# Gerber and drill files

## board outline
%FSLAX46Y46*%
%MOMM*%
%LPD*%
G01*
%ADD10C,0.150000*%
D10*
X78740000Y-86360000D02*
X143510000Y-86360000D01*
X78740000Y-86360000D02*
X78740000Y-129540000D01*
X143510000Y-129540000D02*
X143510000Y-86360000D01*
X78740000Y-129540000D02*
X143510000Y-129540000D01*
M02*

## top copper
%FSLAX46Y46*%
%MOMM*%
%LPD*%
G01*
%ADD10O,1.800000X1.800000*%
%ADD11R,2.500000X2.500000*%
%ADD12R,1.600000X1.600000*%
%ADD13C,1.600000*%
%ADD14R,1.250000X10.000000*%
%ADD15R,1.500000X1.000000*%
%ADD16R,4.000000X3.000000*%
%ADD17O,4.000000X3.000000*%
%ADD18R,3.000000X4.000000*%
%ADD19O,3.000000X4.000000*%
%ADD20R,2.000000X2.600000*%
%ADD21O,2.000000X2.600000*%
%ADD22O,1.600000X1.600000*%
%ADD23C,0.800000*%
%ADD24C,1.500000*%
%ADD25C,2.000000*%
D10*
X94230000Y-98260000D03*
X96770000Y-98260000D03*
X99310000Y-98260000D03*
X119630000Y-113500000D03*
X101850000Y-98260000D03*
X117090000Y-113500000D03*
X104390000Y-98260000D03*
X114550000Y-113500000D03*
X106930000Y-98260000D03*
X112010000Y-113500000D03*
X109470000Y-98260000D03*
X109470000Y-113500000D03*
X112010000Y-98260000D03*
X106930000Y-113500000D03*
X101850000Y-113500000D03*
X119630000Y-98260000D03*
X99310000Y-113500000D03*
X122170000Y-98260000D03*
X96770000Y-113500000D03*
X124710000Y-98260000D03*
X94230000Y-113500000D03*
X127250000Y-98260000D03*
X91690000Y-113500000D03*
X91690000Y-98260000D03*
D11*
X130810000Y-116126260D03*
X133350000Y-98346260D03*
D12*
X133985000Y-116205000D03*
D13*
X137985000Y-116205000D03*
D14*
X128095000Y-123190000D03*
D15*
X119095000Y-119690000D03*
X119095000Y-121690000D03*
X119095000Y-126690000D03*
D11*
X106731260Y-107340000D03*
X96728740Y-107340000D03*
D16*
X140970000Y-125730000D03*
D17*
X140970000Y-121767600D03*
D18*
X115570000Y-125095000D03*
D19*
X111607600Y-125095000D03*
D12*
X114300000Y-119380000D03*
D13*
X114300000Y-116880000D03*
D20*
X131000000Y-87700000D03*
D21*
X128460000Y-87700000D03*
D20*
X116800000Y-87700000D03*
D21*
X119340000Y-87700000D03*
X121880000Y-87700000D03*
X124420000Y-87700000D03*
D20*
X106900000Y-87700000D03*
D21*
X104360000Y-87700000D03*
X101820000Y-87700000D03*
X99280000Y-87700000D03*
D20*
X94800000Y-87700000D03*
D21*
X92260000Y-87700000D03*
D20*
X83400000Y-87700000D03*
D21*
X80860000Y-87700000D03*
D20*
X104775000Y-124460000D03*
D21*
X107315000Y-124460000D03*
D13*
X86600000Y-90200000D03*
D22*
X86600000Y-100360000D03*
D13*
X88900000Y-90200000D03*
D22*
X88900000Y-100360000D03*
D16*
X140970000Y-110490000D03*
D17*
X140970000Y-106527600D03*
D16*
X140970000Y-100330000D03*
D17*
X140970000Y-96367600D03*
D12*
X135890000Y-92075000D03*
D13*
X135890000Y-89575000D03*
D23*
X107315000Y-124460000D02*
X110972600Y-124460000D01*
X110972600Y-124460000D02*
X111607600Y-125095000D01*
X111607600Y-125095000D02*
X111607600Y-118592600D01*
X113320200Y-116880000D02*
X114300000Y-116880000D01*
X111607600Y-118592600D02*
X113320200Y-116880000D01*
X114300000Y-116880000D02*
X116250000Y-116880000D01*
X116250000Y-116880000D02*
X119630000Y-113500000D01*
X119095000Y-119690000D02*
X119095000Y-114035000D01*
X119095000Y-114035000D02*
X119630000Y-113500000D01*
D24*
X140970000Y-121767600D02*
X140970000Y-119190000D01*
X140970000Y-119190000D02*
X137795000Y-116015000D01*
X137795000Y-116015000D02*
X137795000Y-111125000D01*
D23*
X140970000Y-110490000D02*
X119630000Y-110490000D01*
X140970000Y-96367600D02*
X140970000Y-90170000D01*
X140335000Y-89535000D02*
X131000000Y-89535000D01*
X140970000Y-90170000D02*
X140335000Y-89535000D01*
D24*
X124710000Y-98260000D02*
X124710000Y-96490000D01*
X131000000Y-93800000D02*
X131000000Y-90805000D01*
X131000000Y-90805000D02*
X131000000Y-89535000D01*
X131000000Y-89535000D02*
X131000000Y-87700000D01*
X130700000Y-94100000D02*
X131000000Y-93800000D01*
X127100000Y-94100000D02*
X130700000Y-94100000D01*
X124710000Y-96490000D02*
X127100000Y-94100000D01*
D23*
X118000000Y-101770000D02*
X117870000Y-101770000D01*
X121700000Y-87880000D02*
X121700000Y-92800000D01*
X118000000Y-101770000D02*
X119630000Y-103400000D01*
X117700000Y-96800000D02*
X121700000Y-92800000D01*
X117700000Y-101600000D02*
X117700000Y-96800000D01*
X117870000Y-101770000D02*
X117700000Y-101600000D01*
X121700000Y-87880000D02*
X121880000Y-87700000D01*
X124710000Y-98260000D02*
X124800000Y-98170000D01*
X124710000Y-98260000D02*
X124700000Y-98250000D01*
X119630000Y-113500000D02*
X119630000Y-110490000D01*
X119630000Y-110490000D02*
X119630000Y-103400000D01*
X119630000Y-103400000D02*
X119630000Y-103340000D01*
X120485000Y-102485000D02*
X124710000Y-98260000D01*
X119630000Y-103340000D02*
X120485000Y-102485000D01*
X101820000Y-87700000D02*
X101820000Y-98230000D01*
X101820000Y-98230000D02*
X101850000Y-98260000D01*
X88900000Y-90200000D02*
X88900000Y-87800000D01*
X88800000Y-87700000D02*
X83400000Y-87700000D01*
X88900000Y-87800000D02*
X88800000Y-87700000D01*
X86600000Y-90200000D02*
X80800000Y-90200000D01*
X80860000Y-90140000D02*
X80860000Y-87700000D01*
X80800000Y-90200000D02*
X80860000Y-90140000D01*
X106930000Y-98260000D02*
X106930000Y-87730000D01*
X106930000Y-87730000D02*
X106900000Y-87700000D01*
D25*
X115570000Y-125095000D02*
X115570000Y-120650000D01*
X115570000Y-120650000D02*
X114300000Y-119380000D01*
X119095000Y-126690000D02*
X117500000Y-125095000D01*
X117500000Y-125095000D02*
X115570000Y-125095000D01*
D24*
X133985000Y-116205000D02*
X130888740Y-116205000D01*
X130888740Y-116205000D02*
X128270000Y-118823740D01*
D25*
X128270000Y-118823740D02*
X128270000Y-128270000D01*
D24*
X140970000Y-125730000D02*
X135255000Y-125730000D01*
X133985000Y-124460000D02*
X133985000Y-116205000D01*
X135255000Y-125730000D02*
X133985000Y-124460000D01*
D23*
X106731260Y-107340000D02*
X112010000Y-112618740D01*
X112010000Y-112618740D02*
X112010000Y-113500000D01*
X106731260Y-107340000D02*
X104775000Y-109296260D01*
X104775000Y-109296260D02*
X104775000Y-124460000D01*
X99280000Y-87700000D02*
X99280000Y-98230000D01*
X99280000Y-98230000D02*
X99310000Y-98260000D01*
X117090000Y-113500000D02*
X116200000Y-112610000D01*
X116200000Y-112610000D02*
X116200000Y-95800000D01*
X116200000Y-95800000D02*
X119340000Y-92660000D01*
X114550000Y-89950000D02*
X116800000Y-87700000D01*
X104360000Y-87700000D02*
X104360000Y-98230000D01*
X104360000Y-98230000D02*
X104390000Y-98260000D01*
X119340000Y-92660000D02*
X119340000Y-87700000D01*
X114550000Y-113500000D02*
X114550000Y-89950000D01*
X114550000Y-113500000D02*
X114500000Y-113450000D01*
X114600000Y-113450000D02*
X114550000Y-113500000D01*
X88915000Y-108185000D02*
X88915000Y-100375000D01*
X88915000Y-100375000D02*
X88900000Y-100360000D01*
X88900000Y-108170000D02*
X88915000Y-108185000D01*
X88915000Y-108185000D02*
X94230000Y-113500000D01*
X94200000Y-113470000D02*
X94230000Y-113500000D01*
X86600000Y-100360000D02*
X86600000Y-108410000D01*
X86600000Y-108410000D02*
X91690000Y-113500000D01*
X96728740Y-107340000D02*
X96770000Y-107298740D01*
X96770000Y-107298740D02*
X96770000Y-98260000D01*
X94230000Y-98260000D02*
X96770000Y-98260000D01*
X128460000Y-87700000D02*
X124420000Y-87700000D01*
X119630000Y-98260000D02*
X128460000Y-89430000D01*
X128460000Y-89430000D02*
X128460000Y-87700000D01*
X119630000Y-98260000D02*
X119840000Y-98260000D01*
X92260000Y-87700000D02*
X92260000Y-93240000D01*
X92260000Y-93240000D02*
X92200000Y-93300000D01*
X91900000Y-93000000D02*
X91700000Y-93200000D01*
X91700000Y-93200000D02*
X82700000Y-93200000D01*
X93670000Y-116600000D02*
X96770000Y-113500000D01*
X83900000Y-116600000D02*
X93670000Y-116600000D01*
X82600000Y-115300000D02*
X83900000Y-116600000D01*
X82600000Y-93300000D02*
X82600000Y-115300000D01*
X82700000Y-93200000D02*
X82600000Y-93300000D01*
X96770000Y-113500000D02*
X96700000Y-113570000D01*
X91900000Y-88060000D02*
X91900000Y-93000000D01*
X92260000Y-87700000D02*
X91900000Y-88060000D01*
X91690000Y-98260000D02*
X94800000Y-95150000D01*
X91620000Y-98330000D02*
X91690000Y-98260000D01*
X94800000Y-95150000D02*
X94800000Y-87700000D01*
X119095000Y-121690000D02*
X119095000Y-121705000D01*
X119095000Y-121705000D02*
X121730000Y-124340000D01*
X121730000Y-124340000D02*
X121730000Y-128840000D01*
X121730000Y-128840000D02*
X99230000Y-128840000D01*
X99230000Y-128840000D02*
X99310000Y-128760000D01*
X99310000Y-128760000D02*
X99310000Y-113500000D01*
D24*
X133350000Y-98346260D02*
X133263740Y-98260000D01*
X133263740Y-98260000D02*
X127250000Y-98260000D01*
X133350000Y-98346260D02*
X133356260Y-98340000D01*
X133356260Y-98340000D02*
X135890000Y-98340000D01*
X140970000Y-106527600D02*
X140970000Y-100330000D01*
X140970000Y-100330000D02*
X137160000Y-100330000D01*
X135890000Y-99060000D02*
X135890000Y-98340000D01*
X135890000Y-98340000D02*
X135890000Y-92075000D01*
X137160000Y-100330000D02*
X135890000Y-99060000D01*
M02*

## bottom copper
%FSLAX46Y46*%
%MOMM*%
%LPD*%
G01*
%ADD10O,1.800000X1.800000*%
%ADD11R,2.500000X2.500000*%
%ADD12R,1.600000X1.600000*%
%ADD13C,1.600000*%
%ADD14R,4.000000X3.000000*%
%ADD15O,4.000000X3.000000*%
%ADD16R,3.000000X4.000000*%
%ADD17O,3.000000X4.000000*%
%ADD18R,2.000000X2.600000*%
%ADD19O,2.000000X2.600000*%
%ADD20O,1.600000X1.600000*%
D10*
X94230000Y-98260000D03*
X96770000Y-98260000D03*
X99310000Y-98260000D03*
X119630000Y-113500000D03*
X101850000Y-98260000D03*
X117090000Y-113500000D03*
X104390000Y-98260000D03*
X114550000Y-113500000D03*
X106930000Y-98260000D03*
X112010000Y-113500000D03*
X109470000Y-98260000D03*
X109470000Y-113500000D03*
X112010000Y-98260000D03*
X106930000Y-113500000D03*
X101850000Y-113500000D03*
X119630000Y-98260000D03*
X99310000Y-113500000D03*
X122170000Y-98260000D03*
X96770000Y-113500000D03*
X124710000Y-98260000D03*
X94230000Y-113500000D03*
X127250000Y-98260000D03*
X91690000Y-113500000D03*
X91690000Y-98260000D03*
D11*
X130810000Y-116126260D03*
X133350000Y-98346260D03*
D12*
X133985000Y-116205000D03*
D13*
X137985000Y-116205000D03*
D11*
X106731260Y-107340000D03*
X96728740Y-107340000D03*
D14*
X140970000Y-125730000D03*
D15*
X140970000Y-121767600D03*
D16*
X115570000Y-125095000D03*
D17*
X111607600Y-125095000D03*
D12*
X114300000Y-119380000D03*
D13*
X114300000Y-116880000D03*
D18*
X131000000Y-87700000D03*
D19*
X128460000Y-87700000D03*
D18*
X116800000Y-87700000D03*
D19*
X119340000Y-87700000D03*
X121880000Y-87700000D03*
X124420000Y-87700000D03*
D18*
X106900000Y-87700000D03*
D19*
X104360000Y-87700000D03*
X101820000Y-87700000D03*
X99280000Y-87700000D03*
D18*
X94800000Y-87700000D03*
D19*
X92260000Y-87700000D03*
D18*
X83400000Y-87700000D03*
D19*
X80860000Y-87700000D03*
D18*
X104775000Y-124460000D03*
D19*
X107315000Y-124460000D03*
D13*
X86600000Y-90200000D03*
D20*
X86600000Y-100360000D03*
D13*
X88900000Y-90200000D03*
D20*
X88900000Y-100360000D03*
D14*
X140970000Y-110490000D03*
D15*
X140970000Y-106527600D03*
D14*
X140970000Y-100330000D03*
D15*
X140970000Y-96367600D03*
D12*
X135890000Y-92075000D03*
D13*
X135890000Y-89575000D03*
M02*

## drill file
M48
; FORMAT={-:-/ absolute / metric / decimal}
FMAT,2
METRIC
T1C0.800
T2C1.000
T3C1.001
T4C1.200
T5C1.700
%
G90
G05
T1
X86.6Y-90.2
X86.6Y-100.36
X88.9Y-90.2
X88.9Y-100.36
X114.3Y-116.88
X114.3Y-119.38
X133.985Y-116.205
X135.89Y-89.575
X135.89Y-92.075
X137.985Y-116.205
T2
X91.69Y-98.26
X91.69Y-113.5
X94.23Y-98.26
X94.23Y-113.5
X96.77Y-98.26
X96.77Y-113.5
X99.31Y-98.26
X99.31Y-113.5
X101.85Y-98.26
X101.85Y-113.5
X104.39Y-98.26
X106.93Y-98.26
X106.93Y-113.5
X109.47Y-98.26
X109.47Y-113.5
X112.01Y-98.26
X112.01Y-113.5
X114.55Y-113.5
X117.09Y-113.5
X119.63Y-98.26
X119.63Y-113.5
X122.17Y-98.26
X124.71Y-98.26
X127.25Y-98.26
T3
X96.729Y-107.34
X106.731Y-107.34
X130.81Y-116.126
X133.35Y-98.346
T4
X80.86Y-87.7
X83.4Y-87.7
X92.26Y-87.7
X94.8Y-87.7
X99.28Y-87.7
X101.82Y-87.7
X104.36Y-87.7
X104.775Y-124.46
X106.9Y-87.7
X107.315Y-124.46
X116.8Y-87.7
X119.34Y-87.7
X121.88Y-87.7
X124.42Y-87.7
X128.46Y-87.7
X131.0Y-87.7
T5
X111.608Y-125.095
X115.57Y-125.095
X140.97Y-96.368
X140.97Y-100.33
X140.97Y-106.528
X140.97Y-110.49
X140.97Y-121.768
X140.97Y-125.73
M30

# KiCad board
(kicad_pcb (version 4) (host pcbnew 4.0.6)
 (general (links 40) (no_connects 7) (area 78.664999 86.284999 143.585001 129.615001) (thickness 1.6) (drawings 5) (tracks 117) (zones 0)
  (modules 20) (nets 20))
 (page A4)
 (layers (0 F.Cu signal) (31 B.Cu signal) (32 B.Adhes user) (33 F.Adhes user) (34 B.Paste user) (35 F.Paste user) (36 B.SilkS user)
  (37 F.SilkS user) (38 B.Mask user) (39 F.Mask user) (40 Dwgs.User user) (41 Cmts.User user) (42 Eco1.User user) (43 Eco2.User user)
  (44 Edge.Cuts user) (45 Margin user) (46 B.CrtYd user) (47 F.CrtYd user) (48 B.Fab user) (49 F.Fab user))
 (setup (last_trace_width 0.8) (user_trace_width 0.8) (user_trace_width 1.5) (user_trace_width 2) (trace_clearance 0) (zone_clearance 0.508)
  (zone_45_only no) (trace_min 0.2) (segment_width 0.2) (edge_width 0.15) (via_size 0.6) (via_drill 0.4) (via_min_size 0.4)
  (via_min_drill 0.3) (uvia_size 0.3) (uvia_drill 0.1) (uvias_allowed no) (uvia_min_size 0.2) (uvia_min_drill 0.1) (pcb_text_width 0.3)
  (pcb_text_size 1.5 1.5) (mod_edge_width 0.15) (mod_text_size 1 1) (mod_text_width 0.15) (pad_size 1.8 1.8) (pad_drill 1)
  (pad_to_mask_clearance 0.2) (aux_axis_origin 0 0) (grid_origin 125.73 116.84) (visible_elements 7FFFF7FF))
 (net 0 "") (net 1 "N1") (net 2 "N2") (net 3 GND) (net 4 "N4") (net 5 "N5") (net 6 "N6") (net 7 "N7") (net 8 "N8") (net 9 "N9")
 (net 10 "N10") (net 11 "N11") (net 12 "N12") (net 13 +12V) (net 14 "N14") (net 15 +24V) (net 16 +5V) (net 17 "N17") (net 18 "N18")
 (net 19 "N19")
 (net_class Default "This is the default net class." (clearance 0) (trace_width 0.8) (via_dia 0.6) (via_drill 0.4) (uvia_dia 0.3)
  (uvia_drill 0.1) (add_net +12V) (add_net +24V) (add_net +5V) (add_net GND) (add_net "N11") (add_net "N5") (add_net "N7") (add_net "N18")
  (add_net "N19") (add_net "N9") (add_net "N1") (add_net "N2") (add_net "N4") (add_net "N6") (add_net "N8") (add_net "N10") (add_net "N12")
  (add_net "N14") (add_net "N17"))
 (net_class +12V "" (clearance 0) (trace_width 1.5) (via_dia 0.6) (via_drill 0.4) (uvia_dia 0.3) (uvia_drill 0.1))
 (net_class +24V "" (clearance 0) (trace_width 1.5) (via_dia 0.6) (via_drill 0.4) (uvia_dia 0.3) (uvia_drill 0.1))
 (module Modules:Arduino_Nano (layer B.Cu) (at 127.25 113.5 90)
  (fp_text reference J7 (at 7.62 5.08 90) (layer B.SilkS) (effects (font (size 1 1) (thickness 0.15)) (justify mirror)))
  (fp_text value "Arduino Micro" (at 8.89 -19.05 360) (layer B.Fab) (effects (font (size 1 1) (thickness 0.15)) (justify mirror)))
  (pad 3.3V thru_hole oval (at 15.24 -33.02 90) (size 1.8 1.8) (drill 1) (layers *.Cu *.Mask) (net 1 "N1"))
  (pad AREF thru_hole oval (at 15.24 -30.48 90) (size 1.8 1.8) (drill 1) (layers *.Cu *.Mask) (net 1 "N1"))
  (pad A0 thru_hole oval (at 15.24 -27.94 90) (size 1.8 1.8) (drill 1) (layers *.Cu *.Mask) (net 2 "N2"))
  (pad GND thru_hole oval (at 0 -7.62 90) (size 1.8 1.8) (drill 1) (layers *.Cu *.Mask) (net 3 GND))
  (pad A1 thru_hole oval (at 15.24 -25.4 90) (size 1.8 1.8) (drill 1) (layers *.Cu *.Mask) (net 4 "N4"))
  (pad SDA thru_hole oval (at 0 -10.16 90) (size 1.8 1.8) (drill 1) (layers *.Cu *.Mask) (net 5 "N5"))
  (pad A2 thru_hole oval (at 15.24 -22.86 90) (size 1.8 1.8) (drill 1) (layers *.Cu *.Mask) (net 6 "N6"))
  (pad SCL thru_hole oval (at 0 -12.7 90) (size 1.8 1.8) (drill 1) (layers *.Cu *.Mask) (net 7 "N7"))
  (pad A3 thru_hole oval (at 15.24 -20.32 90) (size 1.8 1.8) (drill 1) (layers *.Cu *.Mask) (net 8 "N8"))
  (pad D4 thru_hole oval (at 0 -15.24 90) (size 1.8 1.8) (drill 1) (layers *.Cu *.Mask) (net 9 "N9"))
  (pad A4 thru_hole oval (at 15.24 -17.78 90) (size 1.8 1.8) (drill 1) (layers *.Cu *.Mask) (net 9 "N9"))
  (pad D5 thru_hole oval (at 0 -17.78 90) (size 1.8 1.8) (drill 1) (layers *.Cu *.Mask))
  (pad A5 thru_hole oval (at 15.24 -15.24 90) (size 1.8 1.8) (drill 1) (layers *.Cu *.Mask) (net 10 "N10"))
  (pad D6 thru_hole oval (at 0 -20.32 90) (size 1.8 1.8) (drill 1) (layers *.Cu *.Mask))
  (pad D8 thru_hole oval (at 0 -25.4 90) (size 1.8 1.8) (drill 1) (layers *.Cu *.Mask))
  (pad 5v thru_hole oval (at 15.24 -7.62 90) (size 1.8 1.8) (drill 1) (layers *.Cu *.Mask))
  (pad D9 thru_hole oval (at 0 -27.94 90) (size 1.8 1.8) (drill 1) (layers *.Cu *.Mask) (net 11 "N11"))
  (pad RS thru_hole oval (at 15.24 -5.08 90) (size 1.8 1.8) (drill 1) (layers *.Cu *.Mask))
  (pad D10 thru_hole oval (at 0 -30.48 90) (size 1.8 1.8) (drill 1) (layers *.Cu *.Mask))
  (pad GND thru_hole oval (at 15.24 -2.54 90) (size 1.8 1.8) (drill 1) (layers *.Cu *.Mask) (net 3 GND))
  (pad D11 thru_hole oval (at 0 -33.02 90) (size 1.8 1.8) (drill 1) (layers *.Cu *.Mask) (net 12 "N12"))
  (pad Vin thru_hole oval (at 15.24 0 90) (size 1.8 1.8) (drill 1) (layers *.Cu *.Mask) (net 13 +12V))
  (pad D12 thru_hole oval (at 0 -35.56 90) (size 1.8 1.8) (drill 1) (layers *.Cu *.Mask) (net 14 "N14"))
  (pad D13 thru_hole oval (at 15.24 -35.56 90) (size 1.8 1.8) (drill 1) (layers *.Cu *.Mask)))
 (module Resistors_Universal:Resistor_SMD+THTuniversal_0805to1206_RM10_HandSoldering (layer F.Cu) (at 130.81 111.125 90)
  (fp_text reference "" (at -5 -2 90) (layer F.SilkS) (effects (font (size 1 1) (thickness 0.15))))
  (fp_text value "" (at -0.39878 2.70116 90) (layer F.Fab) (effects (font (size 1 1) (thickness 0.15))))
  (pad 1 thru_hole rect (at -5.00126 0 270) (size 2.5 2.5) (drill 1.00076) (layers *.Cu *.Mask) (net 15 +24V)))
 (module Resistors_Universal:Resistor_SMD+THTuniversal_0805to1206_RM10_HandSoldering (layer F.Cu) (at 133.35 93.345 90)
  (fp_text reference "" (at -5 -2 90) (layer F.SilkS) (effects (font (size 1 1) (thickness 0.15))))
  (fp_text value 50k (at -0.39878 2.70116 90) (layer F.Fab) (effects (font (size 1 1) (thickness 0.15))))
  (pad 1 thru_hole rect (at -5.00126 0 270) (size 2.5 2.5) (drill 1.00076) (layers *.Cu *.Mask) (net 13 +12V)))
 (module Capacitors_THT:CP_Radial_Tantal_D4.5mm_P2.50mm (layer B.Cu) (at 133.985 116.205)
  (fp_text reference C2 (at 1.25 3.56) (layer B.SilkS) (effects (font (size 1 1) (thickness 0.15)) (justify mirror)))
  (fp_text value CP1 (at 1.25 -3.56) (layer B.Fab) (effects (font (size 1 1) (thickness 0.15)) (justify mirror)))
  (pad 1 thru_hole rect (at 0 0) (size 1.6 1.6) (drill 0.8) (layers *.Cu *.Mask) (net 15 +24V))
  (pad 2 thru_hole circle (at 4 0) (size 1.6 1.6) (drill 0.8) (layers *.Cu *.Mask) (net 3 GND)))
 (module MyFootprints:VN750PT (layer F.Cu) (at 125.095 123.19 270)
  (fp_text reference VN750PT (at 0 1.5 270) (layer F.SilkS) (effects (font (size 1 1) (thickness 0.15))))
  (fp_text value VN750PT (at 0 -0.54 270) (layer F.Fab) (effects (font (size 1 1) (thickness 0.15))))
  (pad Vcc smd rect (at 0 -3 270) (size 10 1.25) (layers F.Cu F.Paste F.Mask) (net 15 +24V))
  (pad GND smd rect (at -3.5 6 270) (size 1 1.5) (layers F.Cu F.Paste F.Mask) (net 3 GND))
  (pad Inpu smd rect (at -1.5 6 270) (size 1 1.5) (layers F.Cu F.Paste F.Mask) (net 11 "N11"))
  (pad Vout smd rect (at 3.5 6 270) (size 1 1.5) (layers F.Cu F.Paste F.Mask) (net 15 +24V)))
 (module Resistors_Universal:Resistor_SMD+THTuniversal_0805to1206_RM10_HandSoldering (layer F.Cu) (at 101.73 107.34 180)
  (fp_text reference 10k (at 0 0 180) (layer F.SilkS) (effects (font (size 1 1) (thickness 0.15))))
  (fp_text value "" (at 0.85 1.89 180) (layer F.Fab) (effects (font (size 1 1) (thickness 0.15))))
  (pad 1 thru_hole rect (at -5.00126 0) (size 2.5 2.5) (drill 1.00076) (layers *.Cu *.Mask) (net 9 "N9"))
  (pad 2 thru_hole rect (at 5.00126 0) (size 2.5 2.5) (drill 1.00076) (layers *.Cu *.Mask) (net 1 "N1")))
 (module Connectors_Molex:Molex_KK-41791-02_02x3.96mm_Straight (layer F.Cu) (at 140.97 125.73 90)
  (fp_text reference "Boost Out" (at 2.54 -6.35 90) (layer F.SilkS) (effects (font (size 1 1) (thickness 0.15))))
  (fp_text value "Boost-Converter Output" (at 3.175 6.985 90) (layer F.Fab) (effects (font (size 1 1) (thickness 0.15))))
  (pad 1 thru_hole rect (at 0 0 90) (size 3 4) (drill 1.7) (layers *.Cu *.Mask) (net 15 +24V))
  (pad 2 thru_hole oval (at 3.9624 0 90) (size 3 4) (drill 1.7) (layers *.Cu *.Mask) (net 3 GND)))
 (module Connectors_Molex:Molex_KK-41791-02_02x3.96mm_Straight (layer F.Cu) (at 115.57 125.095 180)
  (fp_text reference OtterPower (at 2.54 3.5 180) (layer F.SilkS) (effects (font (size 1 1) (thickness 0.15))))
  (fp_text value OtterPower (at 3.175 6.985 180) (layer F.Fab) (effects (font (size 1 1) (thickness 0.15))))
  (pad 1 thru_hole rect (at 0 0 180) (size 3 4) (drill 1.7) (layers *.Cu *.Mask) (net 15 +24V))
  (pad 2 thru_hole oval (at 3.9624 0 180) (size 3 4) (drill 1.7) (layers *.Cu *.Mask) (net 3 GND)))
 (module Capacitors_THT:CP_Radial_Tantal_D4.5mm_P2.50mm (layer B.Cu) (at 114.3 119.38 90)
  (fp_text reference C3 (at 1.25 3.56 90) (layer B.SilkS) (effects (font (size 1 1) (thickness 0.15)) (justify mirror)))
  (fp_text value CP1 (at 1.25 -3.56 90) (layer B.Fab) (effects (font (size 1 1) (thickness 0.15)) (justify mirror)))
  (pad + thru_hole rect (at 0 0 90) (size 1.6 1.6) (drill 0.8) (layers *.Cu *.Mask) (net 15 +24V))
  (pad 2 thru_hole circle (at 2.5 0 90) (size 1.6 1.6) (drill 0.8) (layers *.Cu *.Mask) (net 3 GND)))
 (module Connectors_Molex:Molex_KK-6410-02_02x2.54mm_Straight (layer F.Cu) (at 131 87.7 180)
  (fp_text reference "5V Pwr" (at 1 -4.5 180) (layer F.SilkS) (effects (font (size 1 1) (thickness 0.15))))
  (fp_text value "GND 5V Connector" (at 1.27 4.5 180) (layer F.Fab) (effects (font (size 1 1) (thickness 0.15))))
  (pad 1 thru_hole rect (at 0 0 180) (size 2 2.6) (drill 1.2) (layers *.Cu *.Mask) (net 3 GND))
  (pad 2 thru_hole oval (at 2.54 0 180) (size 2 2.6) (drill 1.2) (layers *.Cu *.Mask) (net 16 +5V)))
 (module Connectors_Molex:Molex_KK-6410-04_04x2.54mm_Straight (layer F.Cu) (at 116.8 87.7)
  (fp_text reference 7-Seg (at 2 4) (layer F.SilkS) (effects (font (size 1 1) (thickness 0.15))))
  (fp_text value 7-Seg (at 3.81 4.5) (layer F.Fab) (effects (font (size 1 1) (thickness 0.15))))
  (pad 1 thru_hole rect (at 0 0) (size 2 2.6) (drill 1.2) (layers *.Cu *.Mask) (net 5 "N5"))
  (pad 2 thru_hole oval (at 2.54 0) (size 2 2.6) (drill 1.2) (layers *.Cu *.Mask) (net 7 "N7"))
  (pad 3 thru_hole oval (at 5.08 0) (size 2 2.6) (drill 1.2) (layers *.Cu *.Mask) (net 3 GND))
  (pad 4 thru_hole oval (at 7.62 0) (size 2 2.6) (drill 1.2) (layers *.Cu *.Mask) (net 16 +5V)))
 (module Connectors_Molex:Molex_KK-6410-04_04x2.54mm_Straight (layer F.Cu) (at 106.9 87.7 180)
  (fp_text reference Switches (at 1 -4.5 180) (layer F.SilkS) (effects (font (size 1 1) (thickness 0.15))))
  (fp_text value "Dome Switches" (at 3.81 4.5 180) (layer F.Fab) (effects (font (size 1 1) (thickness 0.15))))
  (pad 1 thru_hole rect (at 0 0 180) (size 2 2.6) (drill 1.2) (layers *.Cu *.Mask) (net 8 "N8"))
  (pad 2 thru_hole oval (at 2.54 0 180) (size 2 2.6) (drill 1.2) (layers *.Cu *.Mask) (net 6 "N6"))
  (pad 3 thru_hole oval (at 5.08 0 180) (size 2 2.6) (drill 1.2) (layers *.Cu *.Mask) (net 4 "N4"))
  (pad 4 thru_hole oval (at 7.62 0 180) (size 2 2.6) (drill 1.2) (layers *.Cu *.Mask) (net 2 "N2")))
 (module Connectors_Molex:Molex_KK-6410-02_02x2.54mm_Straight (layer F.Cu) (at 94.8 87.7 180)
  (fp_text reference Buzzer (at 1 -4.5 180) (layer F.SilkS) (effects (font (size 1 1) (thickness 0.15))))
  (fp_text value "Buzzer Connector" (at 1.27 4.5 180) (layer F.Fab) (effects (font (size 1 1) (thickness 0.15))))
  (pad 1 thru_hole rect (at 0 0 180) (size 2 2.6) (drill 1.2) (layers *.Cu *.Mask) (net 10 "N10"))
  (pad 2 thru_hole oval (at 2.54 0 180) (size 2 2.6) (drill 1.2) (layers *.Cu *.Mask) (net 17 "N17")))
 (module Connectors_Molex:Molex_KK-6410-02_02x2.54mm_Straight (layer F.Cu) (at 83.4 87.7 180)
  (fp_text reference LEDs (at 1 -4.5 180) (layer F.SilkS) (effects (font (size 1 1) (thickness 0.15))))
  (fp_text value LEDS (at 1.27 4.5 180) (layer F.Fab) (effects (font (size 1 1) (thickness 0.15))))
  (pad 1 thru_hole rect (at 0 0 180) (size 2 2.6) (drill 1.2) (layers *.Cu *.Mask) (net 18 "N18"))
  (pad 2 thru_hole oval (at 2.54 0 180) (size 2 2.6) (drill 1.2) (layers *.Cu *.Mask) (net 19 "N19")))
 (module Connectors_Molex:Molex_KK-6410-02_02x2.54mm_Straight (layer F.Cu) (at 104.775 124.46)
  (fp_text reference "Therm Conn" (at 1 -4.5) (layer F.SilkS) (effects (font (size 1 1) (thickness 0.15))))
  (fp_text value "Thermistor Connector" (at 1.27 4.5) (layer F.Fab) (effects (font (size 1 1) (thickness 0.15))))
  (pad 1 thru_hole rect (at 0 0) (size 2 2.6) (drill 1.2) (layers *.Cu *.Mask) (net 9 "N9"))
  (pad 2 thru_hole oval (at 2.54 0) (size 2 2.6) (drill 1.2) (layers *.Cu *.Mask) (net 3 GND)))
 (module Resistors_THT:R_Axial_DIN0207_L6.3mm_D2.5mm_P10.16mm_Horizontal (layer F.Cu) (at 86.6 90.2 270)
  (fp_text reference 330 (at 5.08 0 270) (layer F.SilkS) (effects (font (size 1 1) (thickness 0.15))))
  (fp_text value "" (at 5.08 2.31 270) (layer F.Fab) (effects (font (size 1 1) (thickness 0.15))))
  (pad 1 thru_hole circle (at 0 0 270) (size 1.6 1.6) (drill 0.8) (layers *.Cu *.Mask) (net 19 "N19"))
  (pad 2 thru_hole oval (at 10.16 0 270) (size 1.6 1.6) (drill 0.8) (layers *.Cu *.Mask) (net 14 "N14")))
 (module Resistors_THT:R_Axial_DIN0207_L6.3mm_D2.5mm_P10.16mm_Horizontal (layer F.Cu) (at 88.9 90.2 270)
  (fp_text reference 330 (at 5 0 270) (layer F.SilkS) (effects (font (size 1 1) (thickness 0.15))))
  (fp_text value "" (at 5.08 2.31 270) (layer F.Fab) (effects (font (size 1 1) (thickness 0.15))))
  (pad 1 thru_hole circle (at 0 0 270) (size 1.6 1.6) (drill 0.8) (layers *.Cu *.Mask) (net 18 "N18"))
  (pad 2 thru_hole oval (at 10.16 0 270) (size 1.6 1.6) (drill 0.8) (layers *.Cu *.Mask) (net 12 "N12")))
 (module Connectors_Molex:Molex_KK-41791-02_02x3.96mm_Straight (layer F.Cu) (at 140.97 110.49 90)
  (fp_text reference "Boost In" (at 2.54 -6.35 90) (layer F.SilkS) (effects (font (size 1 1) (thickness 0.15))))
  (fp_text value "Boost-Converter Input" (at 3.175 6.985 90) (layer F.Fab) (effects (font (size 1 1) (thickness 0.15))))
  (pad 1 thru_hole rect (at 0 0 90) (size 3 4) (drill 1.7) (layers *.Cu *.Mask) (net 3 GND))
  (pad 2 thru_hole oval (at 3.9624 0 90) (size 3 4) (drill 1.7) (layers *.Cu *.Mask) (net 13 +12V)))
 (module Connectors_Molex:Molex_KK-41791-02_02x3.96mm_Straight (layer F.Cu) (at 140.97 100.33 90)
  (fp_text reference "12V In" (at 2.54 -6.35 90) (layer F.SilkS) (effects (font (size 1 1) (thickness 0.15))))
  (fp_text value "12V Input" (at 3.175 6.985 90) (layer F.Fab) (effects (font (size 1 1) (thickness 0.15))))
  (pad 1 thru_hole rect (at 0 0 90) (size 3 4) (drill 1.7) (layers *.Cu *.Mask) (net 13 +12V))
  (pad 2 thru_hole oval (at 3.9624 0 90) (size 3 4) (drill 1.7) (layers *.Cu *.Mask) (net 3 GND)))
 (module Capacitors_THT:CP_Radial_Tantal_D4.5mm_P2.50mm (layer F.Cu) (at 135.89 92.075 90)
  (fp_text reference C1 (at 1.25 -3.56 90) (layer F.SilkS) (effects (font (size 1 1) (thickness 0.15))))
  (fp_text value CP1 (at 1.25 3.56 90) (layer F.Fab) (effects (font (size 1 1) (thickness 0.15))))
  (pad 1 thru_hole rect (at 0 0 90) (size 1.6 1.6) (drill 0.8) (layers *.Cu *.Mask) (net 13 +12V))
  (pad 2 thru_hole circle (at 2.5 0 90) (size 1.6 1.6) (drill 0.8) (layers *.Cu *.Mask) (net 3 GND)))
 (gr_line (start 78.74 86.36) (end 143.51 86.36) (angle 90) (layer Edge.Cuts) (width 0.15))
 (gr_line (start 78.74 86.36) (end 78.74 129.54) (angle 90) (layer Edge.Cuts) (width 0.15))
 (gr_line (start 143.51 129.54) (end 143.51 86.36) (angle 90) (layer Edge.Cuts) (width 0.15))
 (gr_line (start 78.74 129.54) (end 143.51 129.54) (angle 90) (layer Edge.Cuts) (width 0.15))
 (segment (start 107.315 124.46) (end 110.9726 124.46) (width 0.8) (layer F.Cu) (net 3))
 (segment (start 110.9726 124.46) (end 111.6076 125.095) (width 0.8) (layer F.Cu) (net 3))
 (segment (start 111.6076 125.095) (end 111.6076 118.5926) (width 0.8) (layer F.Cu) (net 3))
 (segment (start 113.3202 116.88) (end 114.3 116.88) (width 0.8) (layer F.Cu) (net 3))
 (segment (start 111.6076 118.5926) (end 113.3202 116.88) (width 0.8) (layer F.Cu) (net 3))
 (segment (start 114.3 116.88) (end 116.25 116.88) (width 0.8) (layer F.Cu) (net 3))
 (segment (start 116.25 116.88) (end 119.63 113.5) (width 0.8) (layer F.Cu) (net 3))
 (segment (start 119.095 119.69) (end 119.095 114.035) (width 0.8) (layer F.Cu) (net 3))
 (segment (start 119.095 114.035) (end 119.63 113.5) (width 0.8) (layer F.Cu) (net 3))
 (segment (start 140.97 121.7676) (end 140.97 119.19) (width 1.5) (layer F.Cu) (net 3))
 (segment (start 140.97 119.19) (end 137.795 116.015) (width 1.5) (layer F.Cu) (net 3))
 (segment (start 137.795 116.015) (end 137.795 111.125) (width 1.5) (layer F.Cu) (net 3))
 (segment (start 140.97 110.49) (end 119.63 110.49) (width 0.8) (layer F.Cu) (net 3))
 (segment (start 140.97 96.3676) (end 140.97 90.17) (width 0.8) (layer F.Cu) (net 3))
 (segment (start 140.335 89.535) (end 131 89.535) (width 0.8) (layer F.Cu) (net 3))
 (segment (start 140.97 90.17) (end 140.335 89.535) (width 0.8) (layer F.Cu) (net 3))
 (segment (start 124.71 98.26) (end 124.71 96.49) (width 1.5) (layer F.Cu) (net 3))
 (segment (start 131 93.8) (end 131 90.805) (width 1.5) (layer F.Cu) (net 3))
 (segment (start 131 90.805) (end 131 89.535) (width 1.5) (layer F.Cu) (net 3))
 (segment (start 131 89.535) (end 131 87.7) (width 1.5) (layer F.Cu) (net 3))
 (segment (start 130.7 94.1) (end 131 93.8) (width 1.5) (layer F.Cu) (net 3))
 (segment (start 127.1 94.1) (end 130.7 94.1) (width 1.5) (layer F.Cu) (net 3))
 (segment (start 124.71 96.49) (end 127.1 94.1) (width 1.5) (layer F.Cu) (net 3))
 (segment (start 118 101.77) (end 117.87 101.77) (width 0.8) (layer F.Cu) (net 3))
 (segment (start 121.7 87.88) (end 121.7 92.8) (width 0.8) (layer F.Cu) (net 3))
 (segment (start 118 101.77) (end 119.63 103.4) (width 0.8) (layer F.Cu) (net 3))
 (segment (start 117.7 96.8) (end 121.7 92.8) (width 0.8) (layer F.Cu) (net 3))
 (segment (start 117.7 101.6) (end 117.7 96.8) (width 0.8) (layer F.Cu) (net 3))
 (segment (start 117.87 101.77) (end 117.7 101.6) (width 0.8) (layer F.Cu) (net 3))
 (segment (start 121.7 87.88) (end 121.88 87.7) (width 0.8) (layer F.Cu) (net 3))
 (segment (start 124.71 98.26) (end 124.8 98.17) (width 0.8) (layer F.Cu) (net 3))
 (segment (start 124.71 98.26) (end 124.7 98.25) (width 0.8) (layer F.Cu) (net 3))
 (segment (start 119.63 113.5) (end 119.63 110.49) (width 0.8) (layer F.Cu) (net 3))
 (segment (start 119.63 110.49) (end 119.63 103.4) (width 0.8) (layer F.Cu) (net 3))
 (segment (start 119.63 103.4) (end 119.63 103.34) (width 0.8) (layer F.Cu) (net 3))
 (segment (start 120.485 102.485) (end 124.71 98.26) (width 0.8) (layer F.Cu) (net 3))
 (segment (start 119.63 103.34) (end 120.485 102.485) (width 0.8) (layer F.Cu) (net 3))
 (segment (start 101.82 87.7) (end 101.82 98.23) (width 0.8) (layer F.Cu) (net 4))
 (segment (start 101.82 98.23) (end 101.85 98.26) (width 0.8) (layer F.Cu) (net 4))
 (segment (start 88.9 90.2) (end 88.9 87.8) (width 0.8) (layer F.Cu) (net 18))
 (segment (start 88.8 87.7) (end 83.4 87.7) (width 0.8) (layer F.Cu) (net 18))
 (segment (start 88.9 87.8) (end 88.8 87.7) (width 0.8) (layer F.Cu) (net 18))
 (segment (start 86.6 90.2) (end 80.8 90.2) (width 0.8) (layer F.Cu) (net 19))
 (segment (start 80.86 90.14) (end 80.86 87.7) (width 0.8) (layer F.Cu) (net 19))
 (segment (start 80.8 90.2) (end 80.86 90.14) (width 0.8) (layer F.Cu) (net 19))
 (segment (start 106.93 98.26) (end 106.93 87.73) (width 0.8) (layer F.Cu) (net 8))
 (segment (start 106.93 87.73) (end 106.9 87.7) (width 0.8) (layer F.Cu) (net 8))
 (segment (start 115.57 125.095) (end 115.57 120.65) (width 2) (layer F.Cu) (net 15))
 (segment (start 115.57 120.65) (end 114.3 119.38) (width 2) (layer F.Cu) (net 15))
 (segment (start 119.095 126.69) (end 117.5 125.095) (width 2) (layer F.Cu) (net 15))
 (segment (start 117.5 125.095) (end 115.57 125.095) (width 2) (layer F.Cu) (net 15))
 (segment (start 133.985 116.205) (end 130.88874 116.205) (width 1.5) (layer F.Cu) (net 15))
 (segment (start 130.88874 116.205) (end 128.27 118.82374) (width 1.5) (layer F.Cu) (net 15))
 (segment (start 128.27 118.82374) (end 128.27 128.27) (width 2) (layer F.Cu) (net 15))
 (segment (start 140.97 125.73) (end 135.255 125.73) (width 1.5) (layer F.Cu) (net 15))
 (segment (start 133.985 124.46) (end 133.985 116.205) (width 1.5) (layer F.Cu) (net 15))
 (segment (start 135.255 125.73) (end 133.985 124.46) (width 1.5) (layer F.Cu) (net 15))
 (segment (start 106.73126 107.34) (end 112.01 112.61874) (width 0.8) (layer F.Cu) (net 9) (status C00000))
 (segment (start 112.01 112.61874) (end 112.01 113.5) (width 0.8) (layer F.Cu) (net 9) (status C00000))
 (segment (start 106.73126 107.34) (end 104.775 109.29626) (width 0.8) (layer F.Cu) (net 9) (status 400000))
 (segment (start 104.775 109.29626) (end 104.775 124.46) (width 0.8) (layer F.Cu) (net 9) (status 800000))
 (segment (start 99.28 87.7) (end 99.28 98.23) (width 0.8) (layer F.Cu) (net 2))
 (segment (start 99.28 98.23) (end 99.31 98.26) (width 0.8) (layer F.Cu) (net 2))
 (segment (start 117.09 113.5) (end 116.2 112.61) (width 0.8) (layer F.Cu) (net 5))
 (segment (start 116.2 112.61) (end 116.2 95.8) (width 0.8) (layer F.Cu) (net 5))
 (segment (start 116.2 95.8) (end 119.34 92.66) (width 0.8) (layer F.Cu) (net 5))
 (segment (start 114.55 89.95) (end 116.8 87.7) (width 0.8) (layer F.Cu) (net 5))
 (segment (start 104.36 87.7) (end 104.36 98.23) (width 0.8) (layer F.Cu) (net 6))
 (segment (start 104.36 98.23) (end 104.39 98.26) (width 0.8) (layer F.Cu) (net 6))
 (segment (start 119.34 92.66) (end 119.34 87.7) (width 0.8) (layer F.Cu) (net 7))
 (segment (start 114.55 113.5) (end 114.55 89.95) (width 0.8) (layer F.Cu) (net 7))
 (segment (start 114.55 113.5) (end 114.5 113.45) (width 0.8) (layer F.Cu) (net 7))
 (segment (start 114.6 113.45) (end 114.55 113.5) (width 0.8) (layer F.Cu) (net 7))
 (segment (start 88.915 108.185) (end 88.915 100.375) (width 0.8) (layer F.Cu) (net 12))
 (segment (start 88.915 100.375) (end 88.9 100.36) (width 0.8) (layer F.Cu) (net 12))
 (segment (start 88.9 108.17) (end 88.915 108.185) (width 0.8) (layer F.Cu) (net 12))
 (segment (start 88.915 108.185) (end 94.23 113.5) (width 0.8) (layer F.Cu) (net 12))
 (segment (start 94.2 113.47) (end 94.23 113.5) (width 0.8) (layer F.Cu) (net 12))
 (segment (start 86.6 100.36) (end 86.6 108.41) (width 0.8) (layer F.Cu) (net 14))
 (segment (start 86.6 108.41) (end 91.69 113.5) (width 0.8) (layer F.Cu) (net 14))
 (segment (start 96.72874 107.34) (end 96.77 107.29874) (width 0.8) (layer F.Cu) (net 1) (status C00000))
 (segment (start 96.77 107.29874) (end 96.77 98.26) (width 0.8) (layer F.Cu) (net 1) (status C00000))
 (segment (start 94.23 98.26) (end 96.77 98.26) (width 0.8) (layer F.Cu) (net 1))
 (segment (start 128.46 87.7) (end 124.42 87.7) (width 0.8) (layer F.Cu) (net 16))
 (segment (start 119.63 98.26) (end 128.46 89.43) (width 0.8) (layer F.Cu) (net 16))
 (segment (start 128.46 89.43) (end 128.46 87.7) (width 0.8) (layer F.Cu) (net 16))
 (segment (start 119.63 98.26) (end 119.84 98.26) (width 0.8) (layer F.Cu) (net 16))
 (segment (start 92.26 87.7) (end 92.26 93.24) (width 0.8) (layer F.Cu) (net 17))
 (segment (start 92.26 93.24) (end 92.2 93.3) (width 0.8) (layer F.Cu) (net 17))
 (segment (start 91.9 93) (end 91.7 93.2) (width 0.8) (layer F.Cu) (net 17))
 (segment (start 91.7 93.2) (end 82.7 93.2) (width 0.8) (layer F.Cu) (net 17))
 (segment (start 93.67 116.6) (end 96.77 113.5) (width 0.8) (layer F.Cu) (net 17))
 (segment (start 83.9 116.6) (end 93.67 116.6) (width 0.8) (layer F.Cu) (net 17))
 (segment (start 82.6 115.3) (end 83.9 116.6) (width 0.8) (layer F.Cu) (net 17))
 (segment (start 82.6 93.3) (end 82.6 115.3) (width 0.8) (layer F.Cu) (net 17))
 (segment (start 82.7 93.2) (end 82.6 93.3) (width 0.8) (layer F.Cu) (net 17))
 (segment (start 96.77 113.5) (end 96.7 113.57) (width 0.8) (layer F.Cu) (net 17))
 (segment (start 91.9 88.06) (end 91.9 93) (width 0.8) (layer F.Cu) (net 17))
 (segment (start 92.26 87.7) (end 91.9 88.06) (width 0.8) (layer F.Cu) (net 17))
 (segment (start 91.69 98.26) (end 94.8 95.15) (width 0.8) (layer F.Cu) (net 10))
 (segment (start 91.62 98.33) (end 91.69 98.26) (width 0.8) (layer F.Cu) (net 10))
 (segment (start 94.8 95.15) (end 94.8 87.7) (width 0.8) (layer F.Cu) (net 10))
 (segment (start 119.095 121.69) (end 119.095 121.705) (width 0.8) (layer F.Cu) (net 11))
 (segment (start 119.095 121.705) (end 121.73 124.34) (width 0.8) (layer F.Cu) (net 11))
 (segment (start 121.73 124.34) (end 121.73 128.84) (width 0.8) (layer F.Cu) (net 11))
 (segment (start 121.73 128.84) (end 99.23 128.84) (width 0.8) (layer F.Cu) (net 11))
 (segment (start 99.23 128.84) (end 99.31 128.76) (width 0.8) (layer F.Cu) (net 11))
 (segment (start 99.31 128.76) (end 99.31 113.5) (width 0.8) (layer F.Cu) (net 11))
 (segment (start 133.35 98.34626) (end 133.26374 98.26) (width 1.5) (layer F.Cu) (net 13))
 (segment (start 133.26374 98.26) (end 127.25 98.26) (width 1.5) (layer F.Cu) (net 13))
 (segment (start 133.35 98.34626) (end 133.35626 98.34) (width 1.5) (layer F.Cu) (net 13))
 (segment (start 133.35626 98.34) (end 135.89 98.34) (width 1.5) (layer F.Cu) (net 13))
 (segment (start 140.97 106.5276) (end 140.97 100.33) (width 1.5) (layer F.Cu) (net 13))
 (segment (start 140.97 100.33) (end 137.16 100.33) (width 1.5) (layer F.Cu) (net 13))
 (segment (start 135.89 99.06) (end 135.89 98.34) (width 1.5) (layer F.Cu) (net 13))
 (segment (start 135.89 98.34) (end 135.89 92.075) (width 1.5) (layer F.Cu) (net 13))
 (segment (start 137.16 100.33) (end 135.89 99.06) (width 1.5) (layer F.Cu) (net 13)))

